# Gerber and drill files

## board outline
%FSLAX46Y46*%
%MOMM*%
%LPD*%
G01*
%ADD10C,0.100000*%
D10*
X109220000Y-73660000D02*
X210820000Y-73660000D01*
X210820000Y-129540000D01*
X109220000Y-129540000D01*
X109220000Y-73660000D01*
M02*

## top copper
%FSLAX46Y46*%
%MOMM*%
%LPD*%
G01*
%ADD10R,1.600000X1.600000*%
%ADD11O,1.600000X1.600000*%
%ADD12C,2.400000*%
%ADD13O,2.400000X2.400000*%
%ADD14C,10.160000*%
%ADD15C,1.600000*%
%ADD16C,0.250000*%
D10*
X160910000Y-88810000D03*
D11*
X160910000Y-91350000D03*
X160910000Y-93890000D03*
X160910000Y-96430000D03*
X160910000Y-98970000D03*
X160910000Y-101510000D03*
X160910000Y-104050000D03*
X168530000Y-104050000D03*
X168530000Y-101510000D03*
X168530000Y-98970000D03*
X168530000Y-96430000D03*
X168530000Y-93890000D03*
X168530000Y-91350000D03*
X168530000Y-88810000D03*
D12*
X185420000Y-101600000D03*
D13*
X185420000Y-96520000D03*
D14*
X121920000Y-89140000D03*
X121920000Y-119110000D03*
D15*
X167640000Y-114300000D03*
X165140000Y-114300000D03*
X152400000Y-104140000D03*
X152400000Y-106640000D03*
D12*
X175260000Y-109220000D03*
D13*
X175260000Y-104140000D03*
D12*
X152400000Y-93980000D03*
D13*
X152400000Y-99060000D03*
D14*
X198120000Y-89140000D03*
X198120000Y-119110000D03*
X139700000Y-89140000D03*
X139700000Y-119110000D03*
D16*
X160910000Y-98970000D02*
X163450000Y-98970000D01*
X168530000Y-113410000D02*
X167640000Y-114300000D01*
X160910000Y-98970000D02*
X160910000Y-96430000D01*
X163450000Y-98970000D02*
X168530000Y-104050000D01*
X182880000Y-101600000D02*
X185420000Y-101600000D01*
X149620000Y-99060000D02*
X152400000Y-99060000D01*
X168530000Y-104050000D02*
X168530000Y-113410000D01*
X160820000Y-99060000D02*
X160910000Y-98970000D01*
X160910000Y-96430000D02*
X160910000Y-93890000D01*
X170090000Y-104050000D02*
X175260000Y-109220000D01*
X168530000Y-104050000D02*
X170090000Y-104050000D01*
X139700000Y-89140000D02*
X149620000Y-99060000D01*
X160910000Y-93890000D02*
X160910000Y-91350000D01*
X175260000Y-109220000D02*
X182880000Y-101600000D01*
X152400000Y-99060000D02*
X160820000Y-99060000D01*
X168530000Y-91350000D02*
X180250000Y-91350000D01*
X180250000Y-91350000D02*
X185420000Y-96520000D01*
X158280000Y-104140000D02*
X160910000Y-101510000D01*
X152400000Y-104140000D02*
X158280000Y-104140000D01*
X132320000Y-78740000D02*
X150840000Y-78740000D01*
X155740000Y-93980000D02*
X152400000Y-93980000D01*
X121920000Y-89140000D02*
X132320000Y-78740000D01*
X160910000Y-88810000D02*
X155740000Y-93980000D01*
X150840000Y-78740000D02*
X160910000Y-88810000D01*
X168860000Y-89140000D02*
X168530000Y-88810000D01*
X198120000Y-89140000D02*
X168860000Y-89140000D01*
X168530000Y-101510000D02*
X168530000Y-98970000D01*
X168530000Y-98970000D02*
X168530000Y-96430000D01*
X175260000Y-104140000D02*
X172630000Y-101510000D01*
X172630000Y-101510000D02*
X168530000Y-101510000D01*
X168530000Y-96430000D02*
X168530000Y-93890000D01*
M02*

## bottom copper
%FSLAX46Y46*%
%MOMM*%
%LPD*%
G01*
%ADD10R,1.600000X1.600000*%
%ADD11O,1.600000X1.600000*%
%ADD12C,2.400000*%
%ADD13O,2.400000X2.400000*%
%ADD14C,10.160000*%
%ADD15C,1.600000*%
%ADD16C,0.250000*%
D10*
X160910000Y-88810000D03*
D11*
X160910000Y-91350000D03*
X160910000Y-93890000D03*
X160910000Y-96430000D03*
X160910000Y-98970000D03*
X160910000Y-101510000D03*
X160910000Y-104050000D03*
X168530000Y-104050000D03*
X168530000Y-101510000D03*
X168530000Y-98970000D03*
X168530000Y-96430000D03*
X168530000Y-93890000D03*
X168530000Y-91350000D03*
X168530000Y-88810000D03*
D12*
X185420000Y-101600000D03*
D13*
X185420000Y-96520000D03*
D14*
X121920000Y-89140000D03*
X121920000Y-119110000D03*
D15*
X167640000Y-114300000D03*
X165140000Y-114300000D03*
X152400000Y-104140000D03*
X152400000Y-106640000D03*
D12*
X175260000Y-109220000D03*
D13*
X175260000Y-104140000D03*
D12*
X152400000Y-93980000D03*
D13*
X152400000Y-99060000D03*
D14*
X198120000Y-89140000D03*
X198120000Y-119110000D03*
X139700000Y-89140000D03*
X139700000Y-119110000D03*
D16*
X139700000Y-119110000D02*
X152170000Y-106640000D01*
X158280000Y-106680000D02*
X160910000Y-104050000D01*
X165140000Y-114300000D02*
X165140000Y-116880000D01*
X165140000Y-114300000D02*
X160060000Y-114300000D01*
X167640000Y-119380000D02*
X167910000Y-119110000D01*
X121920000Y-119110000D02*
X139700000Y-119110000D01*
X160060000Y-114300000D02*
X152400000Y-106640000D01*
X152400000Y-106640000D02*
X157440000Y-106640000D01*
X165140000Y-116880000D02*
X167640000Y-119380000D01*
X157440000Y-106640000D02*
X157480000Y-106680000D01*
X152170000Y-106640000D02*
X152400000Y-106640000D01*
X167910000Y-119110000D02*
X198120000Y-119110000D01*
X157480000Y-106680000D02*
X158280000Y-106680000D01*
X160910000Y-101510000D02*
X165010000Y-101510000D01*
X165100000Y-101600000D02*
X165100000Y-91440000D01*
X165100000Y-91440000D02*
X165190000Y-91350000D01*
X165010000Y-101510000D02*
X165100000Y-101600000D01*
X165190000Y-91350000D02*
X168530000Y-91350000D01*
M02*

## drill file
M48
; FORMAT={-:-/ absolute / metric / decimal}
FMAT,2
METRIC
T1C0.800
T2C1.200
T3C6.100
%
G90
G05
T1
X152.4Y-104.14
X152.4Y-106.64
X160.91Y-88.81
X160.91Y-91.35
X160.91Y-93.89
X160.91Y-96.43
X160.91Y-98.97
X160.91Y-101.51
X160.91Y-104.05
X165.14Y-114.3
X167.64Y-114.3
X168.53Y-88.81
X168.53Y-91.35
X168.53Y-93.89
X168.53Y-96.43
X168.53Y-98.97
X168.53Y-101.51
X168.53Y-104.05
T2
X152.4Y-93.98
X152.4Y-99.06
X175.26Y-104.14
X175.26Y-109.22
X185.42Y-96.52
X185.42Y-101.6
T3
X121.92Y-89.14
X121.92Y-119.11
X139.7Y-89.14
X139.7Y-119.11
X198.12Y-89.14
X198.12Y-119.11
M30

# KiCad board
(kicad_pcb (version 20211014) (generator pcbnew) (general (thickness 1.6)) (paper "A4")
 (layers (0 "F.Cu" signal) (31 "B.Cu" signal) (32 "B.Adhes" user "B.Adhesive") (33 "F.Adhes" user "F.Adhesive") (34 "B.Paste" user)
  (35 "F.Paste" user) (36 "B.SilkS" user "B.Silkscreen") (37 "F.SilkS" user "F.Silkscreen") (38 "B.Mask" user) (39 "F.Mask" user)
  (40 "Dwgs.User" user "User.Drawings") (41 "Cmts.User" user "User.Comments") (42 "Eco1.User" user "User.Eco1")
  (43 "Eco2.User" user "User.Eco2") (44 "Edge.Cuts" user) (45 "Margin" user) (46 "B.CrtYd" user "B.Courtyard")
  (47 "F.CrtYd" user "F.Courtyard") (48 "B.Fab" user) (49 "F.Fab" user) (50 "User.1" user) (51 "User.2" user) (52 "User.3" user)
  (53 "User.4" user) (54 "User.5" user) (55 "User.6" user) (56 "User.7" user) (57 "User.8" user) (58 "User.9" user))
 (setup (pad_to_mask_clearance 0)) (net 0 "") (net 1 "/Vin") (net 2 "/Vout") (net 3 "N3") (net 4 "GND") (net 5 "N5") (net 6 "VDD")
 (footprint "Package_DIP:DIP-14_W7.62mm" (layer "F.Cu") (at 160.91 88.81)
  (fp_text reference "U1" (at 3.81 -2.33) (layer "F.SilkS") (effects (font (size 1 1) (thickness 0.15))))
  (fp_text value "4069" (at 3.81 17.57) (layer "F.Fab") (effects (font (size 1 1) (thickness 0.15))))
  (pad "1" thru_hole rect (at 0 0) (size 1.6 1.6) (drill 0.8) (layers *.Cu *.Mask) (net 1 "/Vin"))
  (pad "2" thru_hole oval (at 0 2.54) (size 1.6 1.6) (drill 0.8) (layers *.Cu *.Mask) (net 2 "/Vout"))
  (pad "3" thru_hole oval (at 0 5.08) (size 1.6 1.6) (drill 0.8) (layers *.Cu *.Mask) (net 2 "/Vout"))
  (pad "4" thru_hole oval (at 0 7.62) (size 1.6 1.6) (drill 0.8) (layers *.Cu *.Mask) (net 2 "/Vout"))
  (pad "5" thru_hole oval (at 0 10.16) (size 1.6 1.6) (drill 0.8) (layers *.Cu *.Mask) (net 2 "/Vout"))
  (pad "6" thru_hole oval (at 0 12.7) (size 1.6 1.6) (drill 0.8) (layers *.Cu *.Mask) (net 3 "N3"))
  (pad "7" thru_hole oval (at 0 15.24) (size 1.6 1.6) (drill 0.8) (layers *.Cu *.Mask) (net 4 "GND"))
  (pad "8" thru_hole oval (at 7.62 15.24) (size 1.6 1.6) (drill 0.8) (layers *.Cu *.Mask) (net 2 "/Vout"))
  (pad "9" thru_hole oval (at 7.62 12.7) (size 1.6 1.6) (drill 0.8) (layers *.Cu *.Mask) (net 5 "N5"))
  (pad "10" thru_hole oval (at 7.62 10.16) (size 1.6 1.6) (drill 0.8) (layers *.Cu *.Mask) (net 5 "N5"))
  (pad "11" thru_hole oval (at 7.62 7.62) (size 1.6 1.6) (drill 0.8) (layers *.Cu *.Mask) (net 5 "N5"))
  (pad "12" thru_hole oval (at 7.62 5.08) (size 1.6 1.6) (drill 0.8) (layers *.Cu *.Mask) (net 5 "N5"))
  (pad "13" thru_hole oval (at 7.62 2.54) (size 1.6 1.6) (drill 0.8) (layers *.Cu *.Mask) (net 3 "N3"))
  (pad "14" thru_hole oval (at 7.62 0) (size 1.6 1.6) (drill 0.8) (layers *.Cu *.Mask) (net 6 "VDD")))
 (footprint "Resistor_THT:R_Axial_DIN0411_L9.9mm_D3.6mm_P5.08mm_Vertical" (layer "F.Cu") (at 185.42 101.6 90)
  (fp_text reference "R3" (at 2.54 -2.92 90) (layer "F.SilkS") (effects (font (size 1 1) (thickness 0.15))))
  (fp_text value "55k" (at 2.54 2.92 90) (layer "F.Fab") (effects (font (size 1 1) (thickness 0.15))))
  (pad "1" thru_hole circle (at 0 0 90) (size 2.4 2.4) (drill 1.2) (layers *.Cu *.Mask) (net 2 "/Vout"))
  (pad "2" thru_hole oval (at 5.08 0 90) (size 2.4 2.4) (drill 1.2) (layers *.Cu *.Mask) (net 3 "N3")))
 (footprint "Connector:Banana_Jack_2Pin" (layer "F.Cu") (at 121.92 89.14 -90)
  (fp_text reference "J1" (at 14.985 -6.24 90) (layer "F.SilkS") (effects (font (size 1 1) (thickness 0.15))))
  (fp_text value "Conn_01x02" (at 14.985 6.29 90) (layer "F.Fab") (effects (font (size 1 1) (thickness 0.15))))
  (pad "1" thru_hole circle (at 0 0 270) (size 10.16 10.16) (drill 6.1) (layers *.Cu *.Mask) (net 1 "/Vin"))
  (pad "2" thru_hole circle (at 29.97 0 270) (size 10.16 10.16) (drill 6.1) (layers *.Cu *.Mask) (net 4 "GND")))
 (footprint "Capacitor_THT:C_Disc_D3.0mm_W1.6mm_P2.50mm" (layer "F.Cu") (at 167.64 114.3 180)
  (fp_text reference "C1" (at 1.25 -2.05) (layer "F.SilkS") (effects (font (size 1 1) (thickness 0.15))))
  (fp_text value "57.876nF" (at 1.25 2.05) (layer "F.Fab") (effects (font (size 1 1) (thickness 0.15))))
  (pad "1" thru_hole circle (at 0 0 180) (size 1.6 1.6) (drill 0.8) (layers *.Cu *.Mask) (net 2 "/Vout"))
  (pad "2" thru_hole circle (at 2.5 0 180) (size 1.6 1.6) (drill 0.8) (layers *.Cu *.Mask) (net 4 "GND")))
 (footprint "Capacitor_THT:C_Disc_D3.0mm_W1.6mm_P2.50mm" (layer "F.Cu") (at 152.4 104.14 -90)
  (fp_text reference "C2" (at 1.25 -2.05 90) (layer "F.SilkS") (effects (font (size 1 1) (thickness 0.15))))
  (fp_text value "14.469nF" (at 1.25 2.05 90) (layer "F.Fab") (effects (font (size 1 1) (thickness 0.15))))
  (pad "1" thru_hole circle (at 0 0 270) (size 1.6 1.6) (drill 0.8) (layers *.Cu *.Mask) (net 3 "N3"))
  (pad "2" thru_hole circle (at 2.5 0 270) (size 1.6 1.6) (drill 0.8) (layers *.Cu *.Mask) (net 4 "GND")))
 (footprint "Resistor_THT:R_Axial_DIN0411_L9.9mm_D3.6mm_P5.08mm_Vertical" (layer "F.Cu") (at 175.26 109.22 90)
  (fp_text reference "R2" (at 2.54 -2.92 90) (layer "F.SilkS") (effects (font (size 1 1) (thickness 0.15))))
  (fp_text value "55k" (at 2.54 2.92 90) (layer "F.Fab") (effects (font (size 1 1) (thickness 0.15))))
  (pad "1" thru_hole circle (at 0 0 90) (size 2.4 2.4) (drill 1.2) (layers *.Cu *.Mask) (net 2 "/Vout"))
  (pad "2" thru_hole oval (at 5.08 0 90) (size 2.4 2.4) (drill 1.2) (layers *.Cu *.Mask) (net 5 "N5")))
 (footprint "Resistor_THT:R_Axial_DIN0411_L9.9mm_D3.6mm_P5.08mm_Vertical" (layer "F.Cu") (at 152.4 93.98 -90)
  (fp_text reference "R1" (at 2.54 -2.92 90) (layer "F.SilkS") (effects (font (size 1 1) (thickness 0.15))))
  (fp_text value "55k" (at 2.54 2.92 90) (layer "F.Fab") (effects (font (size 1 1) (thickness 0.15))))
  (pad "1" thru_hole circle (at 0 0 270) (size 2.4 2.4) (drill 1.2) (layers *.Cu *.Mask) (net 1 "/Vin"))
  (pad "2" thru_hole oval (at 5.08 0 270) (size 2.4 2.4) (drill 1.2) (layers *.Cu *.Mask) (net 2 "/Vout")))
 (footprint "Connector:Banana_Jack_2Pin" (layer "F.Cu") (at 198.12 89.14 -90)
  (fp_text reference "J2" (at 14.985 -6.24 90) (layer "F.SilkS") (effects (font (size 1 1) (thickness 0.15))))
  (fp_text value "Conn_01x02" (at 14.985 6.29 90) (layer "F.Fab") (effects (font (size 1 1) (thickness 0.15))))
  (pad "1" thru_hole circle (at 0 0 270) (size 10.16 10.16) (drill 6.1) (layers *.Cu *.Mask) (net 6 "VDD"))
  (pad "2" thru_hole circle (at 29.97 0 270) (size 10.16 10.16) (drill 6.1) (layers *.Cu *.Mask) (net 4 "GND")))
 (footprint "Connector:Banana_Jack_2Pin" (layer "F.Cu") (at 139.7 89.14 -90)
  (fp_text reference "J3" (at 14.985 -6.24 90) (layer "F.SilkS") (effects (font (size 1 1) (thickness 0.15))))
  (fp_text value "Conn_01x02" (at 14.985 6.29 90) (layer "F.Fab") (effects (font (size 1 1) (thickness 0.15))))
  (pad "1" thru_hole circle (at 0 0 270) (size 10.16 10.16) (drill 6.1) (layers *.Cu *.Mask) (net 2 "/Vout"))
  (pad "2" thru_hole circle (at 29.97 0 270) (size 10.16 10.16) (drill 6.1) (layers *.Cu *.Mask) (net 4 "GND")))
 (gr_rect (start 109.22 73.66) (end 210.82 129.54) (layer "Edge.Cuts") (width 0.1) (fill none))
 (segment (start 160.91 98.97) (end 163.45 98.97) (width 0.25) (layer "F.Cu") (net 2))
 (segment (start 168.53 113.41) (end 167.64 114.3) (width 0.25) (layer "F.Cu") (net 2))
 (segment (start 160.91 98.97) (end 160.91 96.43) (width 0.25) (layer "F.Cu") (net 2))
 (segment (start 163.45 98.97) (end 168.53 104.05) (width 0.25) (layer "F.Cu") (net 2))
 (segment (start 182.88 101.6) (end 185.42 101.6) (width 0.25) (layer "F.Cu") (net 2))
 (segment (start 149.62 99.06) (end 152.4 99.06) (width 0.25) (layer "F.Cu") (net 2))
 (segment (start 168.53 104.05) (end 168.53 113.41) (width 0.25) (layer "F.Cu") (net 2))
 (segment (start 160.82 99.06) (end 160.91 98.97) (width 0.25) (layer "F.Cu") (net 2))
 (segment (start 160.91 96.43) (end 160.91 93.89) (width 0.25) (layer "F.Cu") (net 2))
 (segment (start 170.09 104.05) (end 175.26 109.22) (width 0.25) (layer "F.Cu") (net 2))
 (segment (start 168.53 104.05) (end 170.09 104.05) (width 0.25) (layer "F.Cu") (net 2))
 (segment (start 139.7 89.14) (end 149.62 99.06) (width 0.25) (layer "F.Cu") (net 2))
 (segment (start 160.91 93.89) (end 160.91 91.35) (width 0.25) (layer "F.Cu") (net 2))
 (segment (start 175.26 109.22) (end 182.88 101.6) (width 0.25) (layer "F.Cu") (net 2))
 (segment (start 152.4 99.06) (end 160.82 99.06) (width 0.25) (layer "F.Cu") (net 2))
 (segment (start 139.7 119.11) (end 152.17 106.64) (width 0.25) (layer "B.Cu") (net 4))
 (segment (start 158.28 106.68) (end 160.91 104.05) (width 0.25) (layer "B.Cu") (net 4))
 (segment (start 165.14 114.3) (end 165.14 116.88) (width 0.25) (layer "B.Cu") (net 4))
 (segment (start 165.14 114.3) (end 160.06 114.3) (width 0.25) (layer "B.Cu") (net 4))
 (segment (start 167.64 119.38) (end 167.91 119.11) (width 0.25) (layer "B.Cu") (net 4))
 (segment (start 121.92 119.11) (end 139.7 119.11) (width 0.25) (layer "B.Cu") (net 4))
 (segment (start 160.06 114.3) (end 152.4 106.64) (width 0.25) (layer "B.Cu") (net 4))
 (segment (start 152.4 106.64) (end 157.44 106.64) (width 0.25) (layer "B.Cu") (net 4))
 (segment (start 165.14 116.88) (end 167.64 119.38) (width 0.25) (layer "B.Cu") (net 4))
 (segment (start 157.44 106.64) (end 157.48 106.68) (width 0.25) (layer "B.Cu") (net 4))
 (segment (start 152.17 106.64) (end 152.4 106.64) (width 0.25) (layer "B.Cu") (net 4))
 (segment (start 167.91 119.11) (end 198.12 119.11) (width 0.25) (layer "B.Cu") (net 4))
 (segment (start 157.48 106.68) (end 158.28 106.68) (width 0.25) (layer "B.Cu") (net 4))
 (segment (start 168.53 91.35) (end 180.25 91.35) (width 0.25) (layer "F.Cu") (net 3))
 (segment (start 180.25 91.35) (end 185.42 96.52) (width 0.25) (layer "F.Cu") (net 3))
 (segment (start 158.28 104.14) (end 160.91 101.51) (width 0.25) (layer "F.Cu") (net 3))
 (segment (start 152.4 104.14) (end 158.28 104.14) (width 0.25) (layer "F.Cu") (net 3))
 (segment (start 160.91 101.51) (end 165.01 101.51) (width 0.25) (layer "B.Cu") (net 3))
 (segment (start 165.1 101.6) (end 165.1 91.44) (width 0.25) (layer "B.Cu") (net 3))
 (segment (start 165.1 91.44) (end 165.19 91.35) (width 0.25) (layer "B.Cu") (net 3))
 (segment (start 165.01 101.51) (end 165.1 101.6) (width 0.25) (layer "B.Cu") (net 3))
 (segment (start 165.19 91.35) (end 168.53 91.35) (width 0.25) (layer "B.Cu") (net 3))
 (segment (start 132.32 78.74) (end 150.84 78.74) (width 0.25) (layer "F.Cu") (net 1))
 (segment (start 155.74 93.98) (end 152.4 93.98) (width 0.25) (layer "F.Cu") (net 1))
 (segment (start 121.92 89.14) (end 132.32 78.74) (width 0.25) (layer "F.Cu") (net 1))
 (segment (start 160.91 88.81) (end 155.74 93.98) (width 0.25) (layer "F.Cu") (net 1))
 (segment (start 150.84 78.74) (end 160.91 88.81) (width 0.25) (layer "F.Cu") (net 1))
 (segment (start 168.86 89.14) (end 168.53 88.81) (width 0.25) (layer "F.Cu") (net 6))
 (segment (start 198.12 89.14) (end 168.86 89.14) (width 0.25) (layer "F.Cu") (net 6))
 (segment (start 168.53 101.51) (end 168.53 98.97) (width 0.25) (layer "F.Cu") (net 5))
 (segment (start 168.53 98.97) (end 168.53 96.43) (width 0.25) (layer "F.Cu") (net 5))
 (segment (start 175.26 104.14) (end 172.63 101.51) (width 0.25) (layer "F.Cu") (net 5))
 (segment (start 172.63 101.51) (end 168.53 101.51) (width 0.25) (layer "F.Cu") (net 5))
 (segment (start 168.53 96.43) (end 168.53 93.89) (width 0.25) (layer "F.Cu") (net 5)))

